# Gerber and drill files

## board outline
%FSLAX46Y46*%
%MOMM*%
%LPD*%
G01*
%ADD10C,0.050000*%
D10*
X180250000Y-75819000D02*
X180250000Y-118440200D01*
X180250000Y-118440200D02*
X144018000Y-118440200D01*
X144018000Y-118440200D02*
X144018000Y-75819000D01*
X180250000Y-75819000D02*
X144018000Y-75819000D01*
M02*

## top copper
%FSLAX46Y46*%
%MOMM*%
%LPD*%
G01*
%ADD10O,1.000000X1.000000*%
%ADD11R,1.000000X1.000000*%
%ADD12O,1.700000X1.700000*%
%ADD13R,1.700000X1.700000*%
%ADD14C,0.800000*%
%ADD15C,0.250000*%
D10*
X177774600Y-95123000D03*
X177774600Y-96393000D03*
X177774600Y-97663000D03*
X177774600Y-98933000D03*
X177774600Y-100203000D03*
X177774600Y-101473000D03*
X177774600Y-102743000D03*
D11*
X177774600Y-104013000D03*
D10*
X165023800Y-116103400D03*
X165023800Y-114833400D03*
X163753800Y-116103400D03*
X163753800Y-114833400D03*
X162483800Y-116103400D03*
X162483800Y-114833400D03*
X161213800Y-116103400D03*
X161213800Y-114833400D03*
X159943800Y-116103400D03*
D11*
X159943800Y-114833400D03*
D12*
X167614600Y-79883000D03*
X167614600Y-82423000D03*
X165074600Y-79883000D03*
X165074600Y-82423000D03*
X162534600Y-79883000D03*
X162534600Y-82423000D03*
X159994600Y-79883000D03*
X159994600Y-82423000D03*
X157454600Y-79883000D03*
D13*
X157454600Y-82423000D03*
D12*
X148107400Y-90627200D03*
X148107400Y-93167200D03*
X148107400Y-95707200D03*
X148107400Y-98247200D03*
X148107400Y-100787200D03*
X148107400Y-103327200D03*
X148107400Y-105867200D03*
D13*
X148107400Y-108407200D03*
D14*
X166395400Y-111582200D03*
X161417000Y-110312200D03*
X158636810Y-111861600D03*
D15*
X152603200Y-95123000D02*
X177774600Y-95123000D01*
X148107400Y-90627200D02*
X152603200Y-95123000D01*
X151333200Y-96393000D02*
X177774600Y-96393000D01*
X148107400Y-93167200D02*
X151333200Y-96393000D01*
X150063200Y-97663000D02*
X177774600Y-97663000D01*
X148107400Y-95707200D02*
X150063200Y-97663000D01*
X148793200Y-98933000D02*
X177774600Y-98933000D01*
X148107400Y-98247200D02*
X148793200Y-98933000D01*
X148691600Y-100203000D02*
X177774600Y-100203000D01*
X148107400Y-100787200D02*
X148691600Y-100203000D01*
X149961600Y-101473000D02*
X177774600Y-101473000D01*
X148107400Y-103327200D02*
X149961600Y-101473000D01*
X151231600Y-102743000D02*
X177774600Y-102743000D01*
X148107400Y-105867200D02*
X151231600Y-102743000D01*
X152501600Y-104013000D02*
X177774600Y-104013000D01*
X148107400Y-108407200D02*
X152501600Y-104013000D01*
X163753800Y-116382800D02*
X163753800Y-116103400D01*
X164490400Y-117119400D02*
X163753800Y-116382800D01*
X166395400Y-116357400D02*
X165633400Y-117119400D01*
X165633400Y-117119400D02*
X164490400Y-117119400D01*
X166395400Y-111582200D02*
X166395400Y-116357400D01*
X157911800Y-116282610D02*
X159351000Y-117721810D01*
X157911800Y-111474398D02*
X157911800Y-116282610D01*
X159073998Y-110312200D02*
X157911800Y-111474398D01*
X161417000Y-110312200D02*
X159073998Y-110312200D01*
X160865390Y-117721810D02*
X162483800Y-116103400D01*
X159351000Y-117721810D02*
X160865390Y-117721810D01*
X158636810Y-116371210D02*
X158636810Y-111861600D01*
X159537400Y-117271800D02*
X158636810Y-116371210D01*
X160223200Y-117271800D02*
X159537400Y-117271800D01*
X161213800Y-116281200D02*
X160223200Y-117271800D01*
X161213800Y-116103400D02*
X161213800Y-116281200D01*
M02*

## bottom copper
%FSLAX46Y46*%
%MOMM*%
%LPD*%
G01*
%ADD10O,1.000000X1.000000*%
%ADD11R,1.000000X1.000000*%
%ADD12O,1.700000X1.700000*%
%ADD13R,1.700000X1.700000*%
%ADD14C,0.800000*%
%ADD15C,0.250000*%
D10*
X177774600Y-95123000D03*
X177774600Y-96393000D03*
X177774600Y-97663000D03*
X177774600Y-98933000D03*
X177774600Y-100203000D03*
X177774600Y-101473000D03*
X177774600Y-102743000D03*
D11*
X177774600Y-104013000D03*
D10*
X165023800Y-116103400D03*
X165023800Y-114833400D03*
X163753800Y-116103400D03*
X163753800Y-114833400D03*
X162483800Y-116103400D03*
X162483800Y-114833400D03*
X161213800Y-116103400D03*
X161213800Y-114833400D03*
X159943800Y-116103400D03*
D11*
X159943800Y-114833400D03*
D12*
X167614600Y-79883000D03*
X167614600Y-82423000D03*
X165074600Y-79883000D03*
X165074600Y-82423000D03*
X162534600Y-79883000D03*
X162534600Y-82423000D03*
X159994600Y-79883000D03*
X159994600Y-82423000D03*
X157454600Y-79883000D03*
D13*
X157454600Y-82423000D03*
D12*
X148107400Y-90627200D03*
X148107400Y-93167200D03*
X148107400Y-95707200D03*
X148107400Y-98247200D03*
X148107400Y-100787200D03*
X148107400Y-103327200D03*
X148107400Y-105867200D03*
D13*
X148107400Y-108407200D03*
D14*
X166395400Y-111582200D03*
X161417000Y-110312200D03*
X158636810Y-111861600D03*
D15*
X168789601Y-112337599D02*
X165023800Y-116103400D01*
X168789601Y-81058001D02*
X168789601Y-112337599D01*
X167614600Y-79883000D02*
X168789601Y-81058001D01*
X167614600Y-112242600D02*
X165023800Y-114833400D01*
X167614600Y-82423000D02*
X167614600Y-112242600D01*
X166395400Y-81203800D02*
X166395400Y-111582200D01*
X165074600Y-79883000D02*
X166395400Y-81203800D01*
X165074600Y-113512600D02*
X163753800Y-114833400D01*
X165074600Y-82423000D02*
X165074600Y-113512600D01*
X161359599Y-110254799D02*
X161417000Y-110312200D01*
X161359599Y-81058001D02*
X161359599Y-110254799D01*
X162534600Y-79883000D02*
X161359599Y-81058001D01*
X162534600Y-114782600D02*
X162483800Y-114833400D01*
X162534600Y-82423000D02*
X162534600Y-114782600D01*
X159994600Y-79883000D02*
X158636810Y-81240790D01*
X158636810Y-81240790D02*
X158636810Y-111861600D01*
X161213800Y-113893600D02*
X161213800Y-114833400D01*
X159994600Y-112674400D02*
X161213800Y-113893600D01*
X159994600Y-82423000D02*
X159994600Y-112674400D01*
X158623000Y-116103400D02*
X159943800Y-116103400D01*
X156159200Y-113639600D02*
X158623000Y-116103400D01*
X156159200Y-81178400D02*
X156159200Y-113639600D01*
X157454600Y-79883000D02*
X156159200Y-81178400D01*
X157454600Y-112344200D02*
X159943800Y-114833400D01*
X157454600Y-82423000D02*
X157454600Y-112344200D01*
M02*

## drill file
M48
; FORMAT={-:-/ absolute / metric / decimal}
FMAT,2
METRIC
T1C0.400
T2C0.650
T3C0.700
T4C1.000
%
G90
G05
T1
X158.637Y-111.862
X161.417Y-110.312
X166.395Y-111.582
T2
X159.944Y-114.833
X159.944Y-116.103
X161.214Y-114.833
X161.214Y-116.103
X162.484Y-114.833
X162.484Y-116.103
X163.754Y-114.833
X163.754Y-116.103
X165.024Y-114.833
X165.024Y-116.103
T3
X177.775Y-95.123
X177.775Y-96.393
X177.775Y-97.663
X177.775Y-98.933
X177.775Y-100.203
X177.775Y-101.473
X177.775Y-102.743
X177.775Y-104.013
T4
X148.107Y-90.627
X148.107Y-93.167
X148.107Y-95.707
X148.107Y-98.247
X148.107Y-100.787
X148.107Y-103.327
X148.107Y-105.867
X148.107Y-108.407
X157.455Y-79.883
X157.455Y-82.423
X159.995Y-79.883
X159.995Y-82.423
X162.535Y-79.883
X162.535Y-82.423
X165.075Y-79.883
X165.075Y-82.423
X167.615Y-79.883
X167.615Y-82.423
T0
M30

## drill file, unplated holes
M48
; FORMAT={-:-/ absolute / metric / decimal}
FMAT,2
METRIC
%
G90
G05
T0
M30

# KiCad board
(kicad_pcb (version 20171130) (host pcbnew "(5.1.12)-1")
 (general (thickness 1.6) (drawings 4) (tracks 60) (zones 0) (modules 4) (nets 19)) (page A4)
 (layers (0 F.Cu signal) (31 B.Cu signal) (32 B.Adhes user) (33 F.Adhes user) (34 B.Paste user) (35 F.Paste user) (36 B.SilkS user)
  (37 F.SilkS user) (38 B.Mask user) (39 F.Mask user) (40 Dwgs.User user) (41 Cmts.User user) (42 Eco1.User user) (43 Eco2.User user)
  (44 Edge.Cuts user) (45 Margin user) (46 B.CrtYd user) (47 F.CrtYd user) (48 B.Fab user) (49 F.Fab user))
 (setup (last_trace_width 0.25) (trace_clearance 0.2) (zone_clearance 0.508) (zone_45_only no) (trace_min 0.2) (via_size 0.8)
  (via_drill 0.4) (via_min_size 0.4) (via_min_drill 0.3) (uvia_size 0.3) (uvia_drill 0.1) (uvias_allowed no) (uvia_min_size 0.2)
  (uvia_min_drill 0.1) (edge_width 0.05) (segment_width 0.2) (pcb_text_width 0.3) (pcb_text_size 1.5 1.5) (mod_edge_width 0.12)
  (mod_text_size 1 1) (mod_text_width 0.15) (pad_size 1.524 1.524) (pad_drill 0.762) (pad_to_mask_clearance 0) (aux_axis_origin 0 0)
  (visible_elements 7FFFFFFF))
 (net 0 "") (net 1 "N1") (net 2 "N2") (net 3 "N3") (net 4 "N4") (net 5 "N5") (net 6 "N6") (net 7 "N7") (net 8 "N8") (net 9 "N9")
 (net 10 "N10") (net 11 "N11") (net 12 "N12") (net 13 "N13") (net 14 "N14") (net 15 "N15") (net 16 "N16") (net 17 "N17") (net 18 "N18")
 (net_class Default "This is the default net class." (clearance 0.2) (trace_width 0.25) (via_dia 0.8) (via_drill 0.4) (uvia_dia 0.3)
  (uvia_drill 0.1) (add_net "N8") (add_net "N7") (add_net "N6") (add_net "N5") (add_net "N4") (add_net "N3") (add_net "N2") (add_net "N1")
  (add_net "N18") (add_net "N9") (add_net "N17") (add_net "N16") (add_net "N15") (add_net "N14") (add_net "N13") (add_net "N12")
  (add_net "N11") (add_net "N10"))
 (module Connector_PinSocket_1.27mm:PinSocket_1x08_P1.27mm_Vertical (layer F.Cu) (at 177.7746 104.013 180)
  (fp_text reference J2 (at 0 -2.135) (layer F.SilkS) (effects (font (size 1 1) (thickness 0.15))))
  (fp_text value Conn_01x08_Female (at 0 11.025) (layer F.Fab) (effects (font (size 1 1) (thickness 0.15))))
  (pad 8 thru_hole oval (at 0 8.89 180) (size 1 1) (drill 0.7) (layers *.Cu *.Mask) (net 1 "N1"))
  (pad 7 thru_hole oval (at 0 7.62 180) (size 1 1) (drill 0.7) (layers *.Cu *.Mask) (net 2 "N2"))
  (pad 6 thru_hole oval (at 0 6.35 180) (size 1 1) (drill 0.7) (layers *.Cu *.Mask) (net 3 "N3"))
  (pad 5 thru_hole oval (at 0 5.08 180) (size 1 1) (drill 0.7) (layers *.Cu *.Mask) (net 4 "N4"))
  (pad 4 thru_hole oval (at 0 3.81 180) (size 1 1) (drill 0.7) (layers *.Cu *.Mask) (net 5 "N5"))
  (pad 3 thru_hole oval (at 0 2.54 180) (size 1 1) (drill 0.7) (layers *.Cu *.Mask) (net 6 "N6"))
  (pad 2 thru_hole oval (at 0 1.27 180) (size 1 1) (drill 0.7) (layers *.Cu *.Mask) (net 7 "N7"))
  (pad 1 thru_hole rect (at 0 0 180) (size 1 1) (drill 0.7) (layers *.Cu *.Mask) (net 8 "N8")))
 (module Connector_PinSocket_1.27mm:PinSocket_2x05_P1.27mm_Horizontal (layer F.Cu) (at 159.9438 114.8334 90)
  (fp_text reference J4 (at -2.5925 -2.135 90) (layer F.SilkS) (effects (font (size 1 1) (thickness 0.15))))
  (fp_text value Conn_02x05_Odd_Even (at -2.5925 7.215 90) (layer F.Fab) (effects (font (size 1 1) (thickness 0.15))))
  (pad 10 thru_hole oval (at -1.27 5.08 90) (size 1 1) (drill 0.65) (layers *.Cu *.Mask) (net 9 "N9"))
  (pad 9 thru_hole oval (at 0 5.08 90) (size 1 1) (drill 0.65) (layers *.Cu *.Mask) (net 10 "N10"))
  (pad 8 thru_hole oval (at -1.27 3.81 90) (size 1 1) (drill 0.65) (layers *.Cu *.Mask) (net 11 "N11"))
  (pad 7 thru_hole oval (at 0 3.81 90) (size 1 1) (drill 0.65) (layers *.Cu *.Mask) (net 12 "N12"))
  (pad 6 thru_hole oval (at -1.27 2.54 90) (size 1 1) (drill 0.65) (layers *.Cu *.Mask) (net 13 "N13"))
  (pad 5 thru_hole oval (at 0 2.54 90) (size 1 1) (drill 0.65) (layers *.Cu *.Mask) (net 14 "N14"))
  (pad 4 thru_hole oval (at -1.27 1.27 90) (size 1 1) (drill 0.65) (layers *.Cu *.Mask) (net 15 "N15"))
  (pad 3 thru_hole oval (at 0 1.27 90) (size 1 1) (drill 0.65) (layers *.Cu *.Mask) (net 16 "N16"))
  (pad 2 thru_hole oval (at -1.27 0 90) (size 1 1) (drill 0.65) (layers *.Cu *.Mask) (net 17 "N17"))
  (pad 1 thru_hole rect (at 0 0 90) (size 1 1) (drill 0.65) (layers *.Cu *.Mask) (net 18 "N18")))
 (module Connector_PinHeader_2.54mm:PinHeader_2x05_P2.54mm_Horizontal (layer F.Cu) (at 157.4546 82.423 90)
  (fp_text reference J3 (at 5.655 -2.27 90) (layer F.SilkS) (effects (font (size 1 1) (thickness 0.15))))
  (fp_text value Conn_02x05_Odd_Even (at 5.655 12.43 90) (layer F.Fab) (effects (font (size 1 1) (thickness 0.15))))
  (pad 10 thru_hole oval (at 2.54 10.16 90) (size 1.7 1.7) (drill 1) (layers *.Cu *.Mask) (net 9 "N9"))
  (pad 9 thru_hole oval (at 0 10.16 90) (size 1.7 1.7) (drill 1) (layers *.Cu *.Mask) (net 10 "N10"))
  (pad 8 thru_hole oval (at 2.54 7.62 90) (size 1.7 1.7) (drill 1) (layers *.Cu *.Mask) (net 11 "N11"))
  (pad 7 thru_hole oval (at 0 7.62 90) (size 1.7 1.7) (drill 1) (layers *.Cu *.Mask) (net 12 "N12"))
  (pad 6 thru_hole oval (at 2.54 5.08 90) (size 1.7 1.7) (drill 1) (layers *.Cu *.Mask) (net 13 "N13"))
  (pad 5 thru_hole oval (at 0 5.08 90) (size 1.7 1.7) (drill 1) (layers *.Cu *.Mask) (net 14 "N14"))
  (pad 4 thru_hole oval (at 2.54 2.54 90) (size 1.7 1.7) (drill 1) (layers *.Cu *.Mask) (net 15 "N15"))
  (pad 3 thru_hole oval (at 0 2.54 90) (size 1.7 1.7) (drill 1) (layers *.Cu *.Mask) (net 16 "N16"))
  (pad 2 thru_hole oval (at 2.54 0 90) (size 1.7 1.7) (drill 1) (layers *.Cu *.Mask) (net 17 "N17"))
  (pad 1 thru_hole rect (at 0 0 90) (size 1.7 1.7) (drill 1) (layers *.Cu *.Mask) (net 18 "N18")))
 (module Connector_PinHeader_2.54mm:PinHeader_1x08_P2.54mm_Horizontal (layer F.Cu) (at 148.1074 108.4072 180)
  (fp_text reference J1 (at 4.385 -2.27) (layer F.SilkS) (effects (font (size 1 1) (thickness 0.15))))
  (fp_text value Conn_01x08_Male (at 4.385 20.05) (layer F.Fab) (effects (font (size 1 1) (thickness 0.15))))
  (pad 8 thru_hole oval (at 0 17.78 180) (size 1.7 1.7) (drill 1) (layers *.Cu *.Mask) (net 1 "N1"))
  (pad 7 thru_hole oval (at 0 15.24 180) (size 1.7 1.7) (drill 1) (layers *.Cu *.Mask) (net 2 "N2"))
  (pad 6 thru_hole oval (at 0 12.7 180) (size 1.7 1.7) (drill 1) (layers *.Cu *.Mask) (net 3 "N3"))
  (pad 5 thru_hole oval (at 0 10.16 180) (size 1.7 1.7) (drill 1) (layers *.Cu *.Mask) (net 4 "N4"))
  (pad 4 thru_hole oval (at 0 7.62 180) (size 1.7 1.7) (drill 1) (layers *.Cu *.Mask) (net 5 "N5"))
  (pad 3 thru_hole oval (at 0 5.08 180) (size 1.7 1.7) (drill 1) (layers *.Cu *.Mask) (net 6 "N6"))
  (pad 2 thru_hole oval (at 0 2.54 180) (size 1.7 1.7) (drill 1) (layers *.Cu *.Mask) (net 7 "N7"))
  (pad 1 thru_hole rect (at 0 0 180) (size 1.7 1.7) (drill 1) (layers *.Cu *.Mask) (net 8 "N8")))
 (gr_line (start 180.25 75.819) (end 180.25 118.4402) (layer Edge.Cuts) (width 0.05))
 (gr_line (start 180.25 118.4402) (end 144.018 118.4402) (layer Edge.Cuts) (width 0.05))
 (gr_line (start 144.018 118.4402) (end 144.018 75.819) (layer Edge.Cuts) (width 0.05))
 (gr_line (start 180.25 75.819) (end 144.018 75.819) (layer Edge.Cuts) (width 0.05))
 (segment (start 152.6032 95.123) (end 177.7746 95.123) (width 0.25) (layer F.Cu) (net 1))
 (segment (start 148.1074 90.6272) (end 152.6032 95.123) (width 0.25) (layer F.Cu) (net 1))
 (segment (start 151.3332 96.393) (end 177.7746 96.393) (width 0.25) (layer F.Cu) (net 2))
 (segment (start 148.1074 93.1672) (end 151.3332 96.393) (width 0.25) (layer F.Cu) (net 2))
 (segment (start 150.0632 97.663) (end 177.7746 97.663) (width 0.25) (layer F.Cu) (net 3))
 (segment (start 148.1074 95.7072) (end 150.0632 97.663) (width 0.25) (layer F.Cu) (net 3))
 (segment (start 148.7932 98.933) (end 177.7746 98.933) (width 0.25) (layer F.Cu) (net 4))
 (segment (start 148.1074 98.2472) (end 148.7932 98.933) (width 0.25) (layer F.Cu) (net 4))
 (segment (start 148.6916 100.203) (end 177.7746 100.203) (width 0.25) (layer F.Cu) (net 5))
 (segment (start 148.1074 100.7872) (end 148.6916 100.203) (width 0.25) (layer F.Cu) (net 5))
 (segment (start 149.9616 101.473) (end 177.7746 101.473) (width 0.25) (layer F.Cu) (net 6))
 (segment (start 148.1074 103.3272) (end 149.9616 101.473) (width 0.25) (layer F.Cu) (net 6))
 (segment (start 151.2316 102.743) (end 177.7746 102.743) (width 0.25) (layer F.Cu) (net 7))
 (segment (start 148.1074 105.8672) (end 151.2316 102.743) (width 0.25) (layer F.Cu) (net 7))
 (segment (start 152.5016 104.013) (end 177.7746 104.013) (width 0.25) (layer F.Cu) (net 8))
 (segment (start 148.1074 108.4072) (end 152.5016 104.013) (width 0.25) (layer F.Cu) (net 8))
 (segment (start 168.789601 112.337599) (end 165.0238 116.1034) (width 0.25) (layer B.Cu) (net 9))
 (segment (start 168.789601 81.058001) (end 168.789601 112.337599) (width 0.25) (layer B.Cu) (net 9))
 (segment (start 167.6146 79.883) (end 168.789601 81.058001) (width 0.25) (layer B.Cu) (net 9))
 (segment (start 167.6146 112.2426) (end 165.0238 114.8334) (width 0.25) (layer B.Cu) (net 10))
 (segment (start 167.6146 82.423) (end 167.6146 112.2426) (width 0.25) (layer B.Cu) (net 10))
 (via (at 166.3954 111.5822) (size 0.8) (drill 0.4) (layers F.Cu B.Cu) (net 11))
 (segment (start 166.3954 81.2038) (end 166.3954 111.5822) (width 0.25) (layer B.Cu) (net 11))
 (segment (start 165.0746 79.883) (end 166.3954 81.2038) (width 0.25) (layer B.Cu) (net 11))
 (segment (start 163.7538 116.3828) (end 163.7538 116.1034) (width 0.25) (layer F.Cu) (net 11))
 (segment (start 164.4904 117.1194) (end 163.7538 116.3828) (width 0.25) (layer F.Cu) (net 11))
 (segment (start 166.3954 116.3574) (end 165.6334 117.1194) (width 0.25) (layer F.Cu) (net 11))
 (segment (start 165.6334 117.1194) (end 164.4904 117.1194) (width 0.25) (layer F.Cu) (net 11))
 (segment (start 166.3954 111.5822) (end 166.3954 116.3574) (width 0.25) (layer F.Cu) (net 11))
 (segment (start 165.0746 113.5126) (end 163.7538 114.8334) (width 0.25) (layer B.Cu) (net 12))
 (segment (start 165.0746 82.423) (end 165.0746 113.5126) (width 0.25) (layer B.Cu) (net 12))
 (via (at 161.417 110.3122) (size 0.8) (drill 0.4) (layers F.Cu B.Cu) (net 13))
 (segment (start 161.359599 110.254799) (end 161.417 110.3122) (width 0.25) (layer B.Cu) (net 13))
 (segment (start 161.359599 81.058001) (end 161.359599 110.254799) (width 0.25) (layer B.Cu) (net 13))
 (segment (start 162.5346 79.883) (end 161.359599 81.058001) (width 0.25) (layer B.Cu) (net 13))
 (segment (start 157.9118 116.28261) (end 159.351 117.72181) (width 0.25) (layer F.Cu) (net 13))
 (segment (start 157.9118 111.474398) (end 157.9118 116.28261) (width 0.25) (layer F.Cu) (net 13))
 (segment (start 159.073998 110.3122) (end 157.9118 111.474398) (width 0.25) (layer F.Cu) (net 13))
 (segment (start 161.417 110.3122) (end 159.073998 110.3122) (width 0.25) (layer F.Cu) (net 13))
 (segment (start 160.86539 117.72181) (end 162.4838 116.1034) (width 0.25) (layer F.Cu) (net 13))
 (segment (start 159.351 117.72181) (end 160.86539 117.72181) (width 0.25) (layer F.Cu) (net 13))
 (segment (start 162.5346 114.7826) (end 162.4838 114.8334) (width 0.25) (layer B.Cu) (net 14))
 (segment (start 162.5346 82.423) (end 162.5346 114.7826) (width 0.25) (layer B.Cu) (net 14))
 (via (at 158.63681 111.8616) (size 0.8) (drill 0.4) (layers F.Cu B.Cu) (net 15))
 (segment (start 159.9946 79.883) (end 158.63681 81.24079) (width 0.25) (layer B.Cu) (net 15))
 (segment (start 158.63681 81.24079) (end 158.63681 111.8616) (width 0.25) (layer B.Cu) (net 15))
 (segment (start 158.63681 116.37121) (end 158.63681 111.8616) (width 0.25) (layer F.Cu) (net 15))
 (segment (start 159.5374 117.2718) (end 158.63681 116.37121) (width 0.25) (layer F.Cu) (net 15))
 (segment (start 160.2232 117.2718) (end 159.5374 117.2718) (width 0.25) (layer F.Cu) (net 15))
 (segment (start 161.2138 116.2812) (end 160.2232 117.2718) (width 0.25) (layer F.Cu) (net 15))
 (segment (start 161.2138 116.1034) (end 161.2138 116.2812) (width 0.25) (layer F.Cu) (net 15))
 (segment (start 161.2138 113.8936) (end 161.2138 114.8334) (width 0.25) (layer B.Cu) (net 16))
 (segment (start 159.9946 112.6744) (end 161.2138 113.8936) (width 0.25) (layer B.Cu) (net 16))
 (segment (start 159.9946 82.423) (end 159.9946 112.6744) (width 0.25) (layer B.Cu) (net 16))
 (segment (start 158.623 116.1034) (end 159.9438 116.1034) (width 0.25) (layer B.Cu) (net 17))
 (segment (start 156.1592 113.6396) (end 158.623 116.1034) (width 0.25) (layer B.Cu) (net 17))
 (segment (start 156.1592 81.1784) (end 156.1592 113.6396) (width 0.25) (layer B.Cu) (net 17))
 (segment (start 157.4546 79.883) (end 156.1592 81.1784) (width 0.25) (layer B.Cu) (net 17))
 (segment (start 157.4546 112.3442) (end 159.9438 114.8334) (width 0.25) (layer B.Cu) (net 18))
 (segment (start 157.4546 82.423) (end 157.4546 112.3442) (width 0.25) (layer B.Cu) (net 18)))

